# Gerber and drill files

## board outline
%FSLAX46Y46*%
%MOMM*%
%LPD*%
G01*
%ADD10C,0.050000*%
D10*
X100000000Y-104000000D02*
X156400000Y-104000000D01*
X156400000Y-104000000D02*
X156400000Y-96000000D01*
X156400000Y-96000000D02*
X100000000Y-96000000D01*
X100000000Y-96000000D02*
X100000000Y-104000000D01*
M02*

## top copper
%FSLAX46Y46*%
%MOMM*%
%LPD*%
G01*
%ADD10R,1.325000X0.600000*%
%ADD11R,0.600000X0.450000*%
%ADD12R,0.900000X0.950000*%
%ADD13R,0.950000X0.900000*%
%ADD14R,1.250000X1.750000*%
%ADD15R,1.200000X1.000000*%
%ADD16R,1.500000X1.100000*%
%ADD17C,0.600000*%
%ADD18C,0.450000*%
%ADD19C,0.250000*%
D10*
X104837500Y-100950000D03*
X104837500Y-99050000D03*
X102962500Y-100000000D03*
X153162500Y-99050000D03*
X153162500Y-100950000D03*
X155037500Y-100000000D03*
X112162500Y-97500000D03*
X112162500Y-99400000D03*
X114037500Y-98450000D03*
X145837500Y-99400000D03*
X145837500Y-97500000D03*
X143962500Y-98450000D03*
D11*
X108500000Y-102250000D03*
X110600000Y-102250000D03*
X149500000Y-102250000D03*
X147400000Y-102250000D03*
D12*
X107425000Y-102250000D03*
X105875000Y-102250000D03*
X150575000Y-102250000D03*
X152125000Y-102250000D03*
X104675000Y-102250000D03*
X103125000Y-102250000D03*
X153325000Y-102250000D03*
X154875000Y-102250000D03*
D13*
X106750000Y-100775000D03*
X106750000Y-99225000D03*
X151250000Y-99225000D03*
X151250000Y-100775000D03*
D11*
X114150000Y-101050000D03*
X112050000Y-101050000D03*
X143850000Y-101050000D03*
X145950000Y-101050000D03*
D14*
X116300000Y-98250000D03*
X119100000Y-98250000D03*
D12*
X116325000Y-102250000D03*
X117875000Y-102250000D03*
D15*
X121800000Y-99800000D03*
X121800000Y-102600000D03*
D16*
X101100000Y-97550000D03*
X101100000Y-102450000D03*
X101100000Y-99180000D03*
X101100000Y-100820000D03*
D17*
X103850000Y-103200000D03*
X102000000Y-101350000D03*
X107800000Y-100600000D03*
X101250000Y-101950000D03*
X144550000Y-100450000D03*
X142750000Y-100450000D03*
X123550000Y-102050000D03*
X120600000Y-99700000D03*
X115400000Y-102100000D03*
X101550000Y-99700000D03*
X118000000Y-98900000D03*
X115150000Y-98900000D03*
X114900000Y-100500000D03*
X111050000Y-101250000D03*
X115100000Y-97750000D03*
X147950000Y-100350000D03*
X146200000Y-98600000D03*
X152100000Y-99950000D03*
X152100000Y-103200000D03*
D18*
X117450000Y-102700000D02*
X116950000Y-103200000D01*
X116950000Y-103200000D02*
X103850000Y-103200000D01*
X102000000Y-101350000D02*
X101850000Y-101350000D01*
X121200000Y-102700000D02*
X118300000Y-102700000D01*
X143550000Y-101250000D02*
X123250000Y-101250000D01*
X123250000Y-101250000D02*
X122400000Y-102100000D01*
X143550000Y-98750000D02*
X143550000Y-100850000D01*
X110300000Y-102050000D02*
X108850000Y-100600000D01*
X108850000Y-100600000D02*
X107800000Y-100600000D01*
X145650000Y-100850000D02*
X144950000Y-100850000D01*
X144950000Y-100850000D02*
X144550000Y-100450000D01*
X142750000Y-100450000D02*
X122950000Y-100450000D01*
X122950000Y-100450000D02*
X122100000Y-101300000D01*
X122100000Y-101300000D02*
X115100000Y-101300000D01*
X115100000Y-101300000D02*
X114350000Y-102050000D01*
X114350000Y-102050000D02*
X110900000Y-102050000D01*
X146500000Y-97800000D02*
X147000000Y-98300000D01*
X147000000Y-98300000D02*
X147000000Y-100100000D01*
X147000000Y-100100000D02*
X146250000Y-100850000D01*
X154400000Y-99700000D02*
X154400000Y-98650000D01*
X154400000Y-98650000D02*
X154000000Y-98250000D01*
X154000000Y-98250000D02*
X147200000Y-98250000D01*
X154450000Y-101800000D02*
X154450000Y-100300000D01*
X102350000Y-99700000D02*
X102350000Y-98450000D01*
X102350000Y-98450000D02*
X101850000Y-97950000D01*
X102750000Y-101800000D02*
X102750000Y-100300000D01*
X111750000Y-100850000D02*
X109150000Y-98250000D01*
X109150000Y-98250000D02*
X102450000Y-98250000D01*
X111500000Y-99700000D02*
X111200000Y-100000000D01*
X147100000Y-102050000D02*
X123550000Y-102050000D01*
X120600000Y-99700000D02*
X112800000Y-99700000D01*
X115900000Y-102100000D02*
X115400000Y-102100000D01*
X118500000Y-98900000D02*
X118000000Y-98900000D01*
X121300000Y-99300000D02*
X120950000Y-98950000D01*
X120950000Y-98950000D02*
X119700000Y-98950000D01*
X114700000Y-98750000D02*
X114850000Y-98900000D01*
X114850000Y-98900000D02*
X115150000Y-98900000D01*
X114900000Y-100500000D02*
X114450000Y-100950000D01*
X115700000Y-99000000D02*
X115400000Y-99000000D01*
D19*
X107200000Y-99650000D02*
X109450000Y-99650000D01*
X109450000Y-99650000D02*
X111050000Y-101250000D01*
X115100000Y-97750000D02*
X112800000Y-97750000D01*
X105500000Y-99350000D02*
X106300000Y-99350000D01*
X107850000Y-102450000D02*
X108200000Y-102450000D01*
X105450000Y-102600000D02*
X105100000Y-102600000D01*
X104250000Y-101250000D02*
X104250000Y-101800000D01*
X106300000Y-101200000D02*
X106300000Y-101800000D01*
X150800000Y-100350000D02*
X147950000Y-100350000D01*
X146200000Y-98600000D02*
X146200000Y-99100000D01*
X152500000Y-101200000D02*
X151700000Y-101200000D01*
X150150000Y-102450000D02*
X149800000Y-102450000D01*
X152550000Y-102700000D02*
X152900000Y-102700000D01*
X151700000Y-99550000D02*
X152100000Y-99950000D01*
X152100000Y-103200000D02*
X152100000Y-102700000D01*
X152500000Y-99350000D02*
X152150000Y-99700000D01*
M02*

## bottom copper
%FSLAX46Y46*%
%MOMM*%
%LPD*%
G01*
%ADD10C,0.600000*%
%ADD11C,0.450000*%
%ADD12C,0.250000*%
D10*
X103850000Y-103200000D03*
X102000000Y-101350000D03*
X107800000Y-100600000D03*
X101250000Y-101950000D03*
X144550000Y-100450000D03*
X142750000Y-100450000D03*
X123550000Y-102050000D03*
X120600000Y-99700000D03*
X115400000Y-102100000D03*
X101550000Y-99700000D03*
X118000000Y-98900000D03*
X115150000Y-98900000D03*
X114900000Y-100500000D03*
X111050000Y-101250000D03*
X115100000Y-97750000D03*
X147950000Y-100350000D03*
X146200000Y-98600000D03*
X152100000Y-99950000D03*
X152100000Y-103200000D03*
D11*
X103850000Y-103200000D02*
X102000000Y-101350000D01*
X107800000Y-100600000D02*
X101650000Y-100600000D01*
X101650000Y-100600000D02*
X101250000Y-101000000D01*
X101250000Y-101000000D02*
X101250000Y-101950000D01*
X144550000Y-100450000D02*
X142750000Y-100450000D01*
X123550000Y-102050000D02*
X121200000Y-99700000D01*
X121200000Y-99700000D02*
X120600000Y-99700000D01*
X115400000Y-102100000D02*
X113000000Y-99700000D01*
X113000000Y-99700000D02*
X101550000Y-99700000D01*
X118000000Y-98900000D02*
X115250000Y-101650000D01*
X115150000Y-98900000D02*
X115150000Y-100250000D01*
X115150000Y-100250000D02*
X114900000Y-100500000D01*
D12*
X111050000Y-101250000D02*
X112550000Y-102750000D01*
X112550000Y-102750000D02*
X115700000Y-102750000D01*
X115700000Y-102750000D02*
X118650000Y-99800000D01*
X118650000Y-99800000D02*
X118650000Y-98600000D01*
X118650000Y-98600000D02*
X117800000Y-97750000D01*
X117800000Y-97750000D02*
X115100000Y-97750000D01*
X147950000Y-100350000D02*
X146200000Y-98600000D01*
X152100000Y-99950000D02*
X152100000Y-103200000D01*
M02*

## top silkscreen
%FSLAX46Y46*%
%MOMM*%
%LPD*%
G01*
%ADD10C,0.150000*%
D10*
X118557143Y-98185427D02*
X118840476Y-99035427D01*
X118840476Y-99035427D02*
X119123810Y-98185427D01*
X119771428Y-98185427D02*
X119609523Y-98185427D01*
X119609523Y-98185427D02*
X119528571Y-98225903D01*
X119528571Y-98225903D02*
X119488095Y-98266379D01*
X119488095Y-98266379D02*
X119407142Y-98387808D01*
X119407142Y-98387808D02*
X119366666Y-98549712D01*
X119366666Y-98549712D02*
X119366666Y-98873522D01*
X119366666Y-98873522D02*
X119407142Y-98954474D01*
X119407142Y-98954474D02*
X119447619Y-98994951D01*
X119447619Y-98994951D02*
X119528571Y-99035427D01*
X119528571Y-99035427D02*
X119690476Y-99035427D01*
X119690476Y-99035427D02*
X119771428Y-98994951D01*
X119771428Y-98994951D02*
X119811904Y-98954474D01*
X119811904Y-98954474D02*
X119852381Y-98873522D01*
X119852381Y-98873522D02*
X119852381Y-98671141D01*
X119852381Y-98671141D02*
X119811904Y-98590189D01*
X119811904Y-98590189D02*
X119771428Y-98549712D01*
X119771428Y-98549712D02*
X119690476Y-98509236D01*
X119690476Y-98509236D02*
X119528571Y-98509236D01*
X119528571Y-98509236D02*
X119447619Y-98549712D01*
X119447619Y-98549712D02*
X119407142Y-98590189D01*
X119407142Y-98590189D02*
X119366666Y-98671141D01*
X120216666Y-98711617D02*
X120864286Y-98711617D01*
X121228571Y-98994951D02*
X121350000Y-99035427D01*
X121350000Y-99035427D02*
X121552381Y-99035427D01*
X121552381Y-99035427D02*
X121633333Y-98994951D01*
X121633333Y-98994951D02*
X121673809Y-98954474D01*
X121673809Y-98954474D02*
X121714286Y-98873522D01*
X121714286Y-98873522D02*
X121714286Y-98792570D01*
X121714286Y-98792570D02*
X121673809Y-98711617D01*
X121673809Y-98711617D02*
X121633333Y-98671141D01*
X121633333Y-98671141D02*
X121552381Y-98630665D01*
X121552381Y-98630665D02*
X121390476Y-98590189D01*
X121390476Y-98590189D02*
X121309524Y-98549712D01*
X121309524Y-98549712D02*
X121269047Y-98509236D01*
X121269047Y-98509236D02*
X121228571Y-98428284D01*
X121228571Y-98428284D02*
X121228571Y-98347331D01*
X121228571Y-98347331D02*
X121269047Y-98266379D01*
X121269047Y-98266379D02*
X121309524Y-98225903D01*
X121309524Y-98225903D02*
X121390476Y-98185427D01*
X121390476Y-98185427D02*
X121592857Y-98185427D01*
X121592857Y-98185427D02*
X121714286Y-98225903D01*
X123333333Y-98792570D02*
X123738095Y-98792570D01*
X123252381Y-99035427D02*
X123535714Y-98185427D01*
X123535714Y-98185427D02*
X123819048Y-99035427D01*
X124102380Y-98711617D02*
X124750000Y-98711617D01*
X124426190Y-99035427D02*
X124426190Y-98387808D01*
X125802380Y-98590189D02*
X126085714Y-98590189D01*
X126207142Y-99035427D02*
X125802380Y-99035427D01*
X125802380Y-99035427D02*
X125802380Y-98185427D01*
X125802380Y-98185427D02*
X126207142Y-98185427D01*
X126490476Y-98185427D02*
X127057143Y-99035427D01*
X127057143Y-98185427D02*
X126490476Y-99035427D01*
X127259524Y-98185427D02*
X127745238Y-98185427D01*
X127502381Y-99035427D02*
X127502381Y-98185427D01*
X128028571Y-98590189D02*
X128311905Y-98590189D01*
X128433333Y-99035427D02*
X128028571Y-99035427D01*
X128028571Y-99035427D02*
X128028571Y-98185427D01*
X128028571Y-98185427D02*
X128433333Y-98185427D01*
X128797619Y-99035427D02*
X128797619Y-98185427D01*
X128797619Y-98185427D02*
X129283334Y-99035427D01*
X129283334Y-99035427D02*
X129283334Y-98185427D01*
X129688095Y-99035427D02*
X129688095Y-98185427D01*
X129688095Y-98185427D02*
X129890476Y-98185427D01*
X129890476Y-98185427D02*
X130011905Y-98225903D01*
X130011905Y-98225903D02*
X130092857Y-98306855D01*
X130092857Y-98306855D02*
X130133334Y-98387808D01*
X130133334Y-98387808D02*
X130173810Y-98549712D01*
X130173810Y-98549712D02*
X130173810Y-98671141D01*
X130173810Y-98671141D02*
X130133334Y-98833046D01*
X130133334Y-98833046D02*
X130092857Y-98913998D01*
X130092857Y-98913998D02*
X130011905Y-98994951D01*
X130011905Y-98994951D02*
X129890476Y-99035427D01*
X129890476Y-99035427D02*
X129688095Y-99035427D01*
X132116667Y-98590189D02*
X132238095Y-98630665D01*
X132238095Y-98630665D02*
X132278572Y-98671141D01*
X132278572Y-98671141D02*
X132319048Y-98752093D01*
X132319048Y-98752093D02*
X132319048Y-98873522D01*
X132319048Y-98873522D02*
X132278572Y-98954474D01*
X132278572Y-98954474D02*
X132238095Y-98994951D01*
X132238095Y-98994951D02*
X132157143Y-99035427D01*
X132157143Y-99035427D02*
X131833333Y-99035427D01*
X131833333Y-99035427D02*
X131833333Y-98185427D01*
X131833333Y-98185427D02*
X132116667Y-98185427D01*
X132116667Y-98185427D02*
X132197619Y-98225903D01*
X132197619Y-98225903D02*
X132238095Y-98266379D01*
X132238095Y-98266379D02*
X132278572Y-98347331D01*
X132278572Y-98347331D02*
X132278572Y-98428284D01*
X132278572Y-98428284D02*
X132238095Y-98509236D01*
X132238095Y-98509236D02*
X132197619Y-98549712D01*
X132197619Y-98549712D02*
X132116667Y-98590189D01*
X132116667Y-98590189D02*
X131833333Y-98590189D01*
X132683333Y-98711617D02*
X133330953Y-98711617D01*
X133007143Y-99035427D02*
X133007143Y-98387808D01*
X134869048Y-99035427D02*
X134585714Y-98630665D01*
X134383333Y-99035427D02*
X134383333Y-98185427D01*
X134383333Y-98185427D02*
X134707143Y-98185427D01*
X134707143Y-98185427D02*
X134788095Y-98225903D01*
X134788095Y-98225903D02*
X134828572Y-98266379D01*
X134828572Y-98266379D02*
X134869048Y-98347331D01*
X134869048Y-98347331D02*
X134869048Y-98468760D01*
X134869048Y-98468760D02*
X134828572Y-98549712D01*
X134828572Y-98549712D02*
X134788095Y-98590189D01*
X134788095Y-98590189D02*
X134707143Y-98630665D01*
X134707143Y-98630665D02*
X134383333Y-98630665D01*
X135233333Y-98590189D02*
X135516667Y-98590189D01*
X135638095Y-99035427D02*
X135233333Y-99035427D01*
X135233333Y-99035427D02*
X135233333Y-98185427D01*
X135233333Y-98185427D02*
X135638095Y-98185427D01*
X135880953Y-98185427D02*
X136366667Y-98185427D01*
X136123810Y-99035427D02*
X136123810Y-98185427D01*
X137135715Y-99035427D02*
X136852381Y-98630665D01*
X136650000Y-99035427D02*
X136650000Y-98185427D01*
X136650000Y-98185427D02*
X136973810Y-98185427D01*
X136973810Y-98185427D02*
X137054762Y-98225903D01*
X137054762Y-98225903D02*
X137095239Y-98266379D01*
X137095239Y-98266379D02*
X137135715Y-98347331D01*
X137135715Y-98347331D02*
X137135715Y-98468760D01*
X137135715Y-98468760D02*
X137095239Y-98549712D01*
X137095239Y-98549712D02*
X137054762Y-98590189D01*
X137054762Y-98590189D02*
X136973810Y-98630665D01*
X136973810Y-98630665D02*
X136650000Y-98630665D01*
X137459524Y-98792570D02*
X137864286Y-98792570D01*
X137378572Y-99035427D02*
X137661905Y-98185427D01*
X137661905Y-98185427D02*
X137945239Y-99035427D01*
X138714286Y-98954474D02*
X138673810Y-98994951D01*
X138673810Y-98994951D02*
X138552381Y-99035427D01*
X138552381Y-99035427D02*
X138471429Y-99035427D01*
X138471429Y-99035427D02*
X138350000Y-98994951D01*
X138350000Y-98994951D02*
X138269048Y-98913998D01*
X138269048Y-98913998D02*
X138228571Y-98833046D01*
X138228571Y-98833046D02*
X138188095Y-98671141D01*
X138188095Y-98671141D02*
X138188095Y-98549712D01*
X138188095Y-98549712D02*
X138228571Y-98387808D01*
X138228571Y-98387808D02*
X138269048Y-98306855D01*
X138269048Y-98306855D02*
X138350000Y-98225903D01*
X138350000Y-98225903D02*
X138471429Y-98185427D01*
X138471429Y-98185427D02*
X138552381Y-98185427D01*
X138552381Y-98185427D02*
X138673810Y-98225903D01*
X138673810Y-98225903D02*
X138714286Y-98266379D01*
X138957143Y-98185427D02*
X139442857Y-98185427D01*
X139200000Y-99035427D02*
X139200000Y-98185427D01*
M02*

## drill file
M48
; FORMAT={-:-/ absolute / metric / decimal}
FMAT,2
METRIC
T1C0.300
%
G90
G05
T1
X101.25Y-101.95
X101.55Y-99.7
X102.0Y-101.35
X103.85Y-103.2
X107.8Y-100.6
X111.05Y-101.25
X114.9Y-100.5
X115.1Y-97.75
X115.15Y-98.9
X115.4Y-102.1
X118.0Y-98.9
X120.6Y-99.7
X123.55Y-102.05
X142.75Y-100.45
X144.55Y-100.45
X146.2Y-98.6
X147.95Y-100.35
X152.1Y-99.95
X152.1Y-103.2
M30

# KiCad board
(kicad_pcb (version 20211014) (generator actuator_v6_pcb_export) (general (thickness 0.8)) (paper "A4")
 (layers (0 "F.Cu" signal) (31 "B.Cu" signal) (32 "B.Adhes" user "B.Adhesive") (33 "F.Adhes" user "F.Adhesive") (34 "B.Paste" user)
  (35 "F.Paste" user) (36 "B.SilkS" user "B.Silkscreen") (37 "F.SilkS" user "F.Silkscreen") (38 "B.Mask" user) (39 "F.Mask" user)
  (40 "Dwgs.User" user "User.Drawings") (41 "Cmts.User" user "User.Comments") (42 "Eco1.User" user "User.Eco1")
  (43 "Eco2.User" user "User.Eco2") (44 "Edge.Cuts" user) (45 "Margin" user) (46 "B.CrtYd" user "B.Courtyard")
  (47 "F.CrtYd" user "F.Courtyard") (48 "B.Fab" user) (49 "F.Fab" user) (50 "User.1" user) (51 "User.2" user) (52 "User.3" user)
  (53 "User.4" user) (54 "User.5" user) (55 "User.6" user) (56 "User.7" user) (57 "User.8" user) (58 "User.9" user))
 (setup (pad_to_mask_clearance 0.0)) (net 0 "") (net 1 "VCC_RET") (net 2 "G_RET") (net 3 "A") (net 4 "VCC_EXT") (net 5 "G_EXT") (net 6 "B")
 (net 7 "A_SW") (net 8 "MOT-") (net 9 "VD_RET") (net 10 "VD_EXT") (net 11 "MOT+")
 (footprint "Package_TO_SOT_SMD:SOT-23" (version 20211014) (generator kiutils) (layer "F.Cu") (at 103.9 100.0 180)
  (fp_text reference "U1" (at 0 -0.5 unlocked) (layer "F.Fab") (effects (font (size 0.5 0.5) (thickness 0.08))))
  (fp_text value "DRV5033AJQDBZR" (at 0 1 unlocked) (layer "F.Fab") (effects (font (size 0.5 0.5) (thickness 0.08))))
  (pad "1" smd rect (at -0.9375 -0.95 180) (size 1.325 0.6) (layers "F.Cu" "F.Mask" "F.Paste") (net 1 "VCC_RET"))
  (pad "2" smd rect (at -0.9375 0.95 180) (size 1.325 0.6) (layers "F.Cu" "F.Mask" "F.Paste") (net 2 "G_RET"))
  (pad "3" smd rect (at 0.9375 0.0 180) (size 1.325 0.6) (layers "F.Cu" "F.Mask" "F.Paste") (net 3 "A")))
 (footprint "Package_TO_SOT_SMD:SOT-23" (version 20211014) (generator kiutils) (layer "F.Cu") (at 154.1 100.0)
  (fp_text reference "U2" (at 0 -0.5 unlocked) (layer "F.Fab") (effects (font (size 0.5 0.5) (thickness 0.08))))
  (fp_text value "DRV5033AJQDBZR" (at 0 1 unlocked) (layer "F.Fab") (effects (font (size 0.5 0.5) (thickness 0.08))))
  (pad "1" smd rect (at -0.9375 -0.95) (size 1.325 0.6) (layers "F.Cu" "F.Mask" "F.Paste") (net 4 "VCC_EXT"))
  (pad "2" smd rect (at -0.9375 0.95) (size 1.325 0.6) (layers "F.Cu" "F.Mask" "F.Paste") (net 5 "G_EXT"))
  (pad "3" smd rect (at 0.9375 0.0) (size 1.325 0.6) (layers "F.Cu" "F.Mask" "F.Paste") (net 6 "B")))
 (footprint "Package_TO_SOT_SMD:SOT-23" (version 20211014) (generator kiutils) (layer "F.Cu") (at 113.1 98.45)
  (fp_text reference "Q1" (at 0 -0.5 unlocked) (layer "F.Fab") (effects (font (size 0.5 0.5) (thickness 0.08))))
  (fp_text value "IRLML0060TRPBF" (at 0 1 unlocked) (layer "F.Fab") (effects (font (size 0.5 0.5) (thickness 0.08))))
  (pad "1" smd rect (at -0.9375 -0.95) (size 1.325 0.6) (layers "F.Cu" "F.Mask" "F.Paste") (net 2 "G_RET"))
  (pad "2" smd rect (at -0.9375 0.95) (size 1.325 0.6) (layers "F.Cu" "F.Mask" "F.Paste") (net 3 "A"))
  (pad "3" smd rect (at 0.9375 0.0) (size 1.325 0.6) (layers "F.Cu" "F.Mask" "F.Paste") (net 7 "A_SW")))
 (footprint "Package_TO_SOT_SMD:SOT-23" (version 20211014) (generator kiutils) (layer "F.Cu") (at 144.9 98.45 180)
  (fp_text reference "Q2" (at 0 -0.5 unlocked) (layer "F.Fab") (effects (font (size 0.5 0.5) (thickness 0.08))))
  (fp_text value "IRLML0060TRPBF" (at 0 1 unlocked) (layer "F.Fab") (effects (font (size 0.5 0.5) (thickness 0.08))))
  (pad "1" smd rect (at -0.9375 -0.95 180) (size 1.325 0.6) (layers "F.Cu" "F.Mask" "F.Paste") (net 5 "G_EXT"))
  (pad "2" smd rect (at -0.9375 0.95 180) (size 1.325 0.6) (layers "F.Cu" "F.Mask" "F.Paste") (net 6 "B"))
  (pad "3" smd rect (at 0.9375 0.0 180) (size 1.325 0.6) (layers "F.Cu" "F.Mask" "F.Paste") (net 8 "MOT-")))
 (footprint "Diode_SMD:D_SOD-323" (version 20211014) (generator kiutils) (layer "F.Cu") (at 109.55 102.25)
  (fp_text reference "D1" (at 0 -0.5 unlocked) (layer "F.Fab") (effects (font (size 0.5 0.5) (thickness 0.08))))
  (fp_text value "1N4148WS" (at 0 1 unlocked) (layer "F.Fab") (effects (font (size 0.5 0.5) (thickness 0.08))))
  (pad "1" smd rect (at -1.05 0.0) (size 0.6 0.45) (layers "F.Cu" "F.Mask" "F.Paste") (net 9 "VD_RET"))
  (pad "2" smd rect (at 1.05 0.0) (size 0.6 0.45) (layers "F.Cu" "F.Mask" "F.Paste") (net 6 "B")))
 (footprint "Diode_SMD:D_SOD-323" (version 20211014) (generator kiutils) (layer "F.Cu") (at 148.45 102.25 180)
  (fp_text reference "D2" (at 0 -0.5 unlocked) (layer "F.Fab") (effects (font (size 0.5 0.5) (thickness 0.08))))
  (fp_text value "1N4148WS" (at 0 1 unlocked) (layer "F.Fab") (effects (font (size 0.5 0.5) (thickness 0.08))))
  (pad "1" smd rect (at -1.05 0.0 180) (size 0.6 0.45) (layers "F.Cu" "F.Mask" "F.Paste") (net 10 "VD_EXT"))
  (pad "2" smd rect (at 1.05 0.0 180) (size 0.6 0.45) (layers "F.Cu" "F.Mask" "F.Paste") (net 3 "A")))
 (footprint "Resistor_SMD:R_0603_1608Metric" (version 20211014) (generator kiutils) (layer "F.Cu") (at 106.65 102.25 180)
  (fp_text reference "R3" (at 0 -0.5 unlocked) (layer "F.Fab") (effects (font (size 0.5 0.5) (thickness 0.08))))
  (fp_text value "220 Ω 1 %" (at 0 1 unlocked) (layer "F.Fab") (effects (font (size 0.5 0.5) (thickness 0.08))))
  (pad "1" smd rect (at -0.775 0.0 180) (size 0.9 0.95) (layers "F.Cu" "F.Mask" "F.Paste") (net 9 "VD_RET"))
  (pad "2" smd rect (at 0.775 0.0 180) (size 0.9 0.95) (layers "F.Cu" "F.Mask" "F.Paste") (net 1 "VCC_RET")))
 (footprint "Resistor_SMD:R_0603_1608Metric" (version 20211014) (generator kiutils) (layer "F.Cu") (at 151.35 102.25)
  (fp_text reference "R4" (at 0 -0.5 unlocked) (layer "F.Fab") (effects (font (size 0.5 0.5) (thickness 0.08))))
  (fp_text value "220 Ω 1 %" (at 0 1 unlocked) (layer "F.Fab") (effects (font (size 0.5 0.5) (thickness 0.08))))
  (pad "1" smd rect (at -0.775 0.0) (size 0.9 0.95) (layers "F.Cu" "F.Mask" "F.Paste") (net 10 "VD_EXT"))
  (pad "2" smd rect (at 0.775 0.0) (size 0.9 0.95) (layers "F.Cu" "F.Mask" "F.Paste") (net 4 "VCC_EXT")))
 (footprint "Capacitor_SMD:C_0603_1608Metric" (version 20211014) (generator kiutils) (layer "F.Cu") (at 103.9 102.25 180)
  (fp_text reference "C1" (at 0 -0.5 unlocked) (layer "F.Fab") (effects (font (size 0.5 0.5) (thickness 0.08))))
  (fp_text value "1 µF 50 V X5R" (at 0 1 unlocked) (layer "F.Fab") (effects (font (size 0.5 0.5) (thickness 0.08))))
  (pad "1" smd rect (at -0.775 0.0 180) (size 0.9 0.95) (layers "F.Cu" "F.Mask" "F.Paste") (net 1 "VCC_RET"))
  (pad "2" smd rect (at 0.775 0.0 180) (size 0.9 0.95) (layers "F.Cu" "F.Mask" "F.Paste") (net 3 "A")))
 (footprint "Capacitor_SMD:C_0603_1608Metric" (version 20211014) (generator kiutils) (layer "F.Cu") (at 154.1 102.25)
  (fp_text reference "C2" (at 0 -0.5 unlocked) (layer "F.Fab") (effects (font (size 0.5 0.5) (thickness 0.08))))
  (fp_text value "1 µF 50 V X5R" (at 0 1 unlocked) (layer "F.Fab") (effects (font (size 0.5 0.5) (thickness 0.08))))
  (pad "1" smd rect (at -0.775 0.0) (size 0.9 0.95) (layers "F.Cu" "F.Mask" "F.Paste") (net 4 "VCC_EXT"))
  (pad "2" smd rect (at 0.775 0.0) (size 0.9 0.95) (layers "F.Cu" "F.Mask" "F.Paste") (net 6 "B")))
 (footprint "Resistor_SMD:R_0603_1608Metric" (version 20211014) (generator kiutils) (layer "F.Cu") (at 106.75 100.0 90)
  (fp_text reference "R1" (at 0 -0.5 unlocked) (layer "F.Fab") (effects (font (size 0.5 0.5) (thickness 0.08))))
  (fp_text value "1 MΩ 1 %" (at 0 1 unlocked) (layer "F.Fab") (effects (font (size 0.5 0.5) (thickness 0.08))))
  (pad "1" smd rect (at -0.775 0.0 90) (size 0.9 0.95) (layers "F.Cu" "F.Mask" "F.Paste") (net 1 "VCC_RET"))
  (pad "2" smd rect (at 0.775 0.0 90) (size 0.9 0.95) (layers "F.Cu" "F.Mask" "F.Paste") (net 2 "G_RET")))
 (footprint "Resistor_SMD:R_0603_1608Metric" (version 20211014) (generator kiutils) (layer "F.Cu") (at 151.25 100.0 270)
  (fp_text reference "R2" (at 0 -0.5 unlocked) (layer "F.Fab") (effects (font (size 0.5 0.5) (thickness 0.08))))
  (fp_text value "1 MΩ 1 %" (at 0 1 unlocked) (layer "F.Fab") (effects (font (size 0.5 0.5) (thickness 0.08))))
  (pad "1" smd rect (at -0.775 0.0 270) (size 0.9 0.95) (layers "F.Cu" "F.Mask" "F.Paste") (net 4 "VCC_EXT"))
  (pad "2" smd rect (at 0.775 0.0 270) (size 0.9 0.95) (layers "F.Cu" "F.Mask" "F.Paste") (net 5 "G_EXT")))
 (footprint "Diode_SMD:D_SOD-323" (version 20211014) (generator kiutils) (layer "F.Cu") (at 113.1 101.05 180)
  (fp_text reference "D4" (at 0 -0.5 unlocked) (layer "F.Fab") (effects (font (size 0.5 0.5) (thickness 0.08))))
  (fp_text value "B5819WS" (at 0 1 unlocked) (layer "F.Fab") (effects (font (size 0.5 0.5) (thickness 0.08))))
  (pad "1" smd rect (at -1.05 0.0 180) (size 0.6 0.45) (layers "F.Cu" "F.Mask" "F.Paste") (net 7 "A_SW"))
  (pad "2" smd rect (at 1.05 0.0 180) (size 0.6 0.45) (layers "F.Cu" "F.Mask" "F.Paste") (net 3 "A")))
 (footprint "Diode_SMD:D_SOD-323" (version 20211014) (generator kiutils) (layer "F.Cu") (at 144.9 101.05)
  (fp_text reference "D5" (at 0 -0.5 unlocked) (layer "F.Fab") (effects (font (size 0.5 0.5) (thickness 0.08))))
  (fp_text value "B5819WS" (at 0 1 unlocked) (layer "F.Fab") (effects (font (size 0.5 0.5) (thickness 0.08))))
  (pad "1" smd rect (at -1.05 0.0) (size 0.6 0.45) (layers "F.Cu" "F.Mask" "F.Paste") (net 8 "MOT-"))
  (pad "2" smd rect (at 1.05 0.0) (size 0.6 0.45) (layers "F.Cu" "F.Mask" "F.Paste") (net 6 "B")))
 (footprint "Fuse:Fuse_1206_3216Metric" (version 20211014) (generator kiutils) (layer "F.Cu") (at 117.7 98.25)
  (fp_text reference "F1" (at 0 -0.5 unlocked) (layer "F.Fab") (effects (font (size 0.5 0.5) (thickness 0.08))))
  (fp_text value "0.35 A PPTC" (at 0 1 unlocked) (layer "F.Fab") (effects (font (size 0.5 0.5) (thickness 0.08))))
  (pad "1" smd rect (at -1.4 0.0) (size 1.25 1.75) (layers "F.Cu" "F.Mask" "F.Paste") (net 7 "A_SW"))
  (pad "2" smd rect (at 1.4 0.0) (size 1.25 1.75) (layers "F.Cu" "F.Mask" "F.Paste") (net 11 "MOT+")))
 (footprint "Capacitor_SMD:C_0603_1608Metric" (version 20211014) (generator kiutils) (layer "F.Cu") (at 117.1 102.25)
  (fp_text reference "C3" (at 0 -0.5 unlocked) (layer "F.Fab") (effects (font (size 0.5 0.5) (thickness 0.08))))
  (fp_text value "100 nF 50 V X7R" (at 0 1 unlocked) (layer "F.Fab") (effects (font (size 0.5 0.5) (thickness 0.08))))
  (pad "1" smd rect (at -0.775 0.0) (size 0.9 0.95) (layers "F.Cu" "F.Mask" "F.Paste") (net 11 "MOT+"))
  (pad "2" smd rect (at 0.775 0.0) (size 0.9 0.95) (layers "F.Cu" "F.Mask" "F.Paste") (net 8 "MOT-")))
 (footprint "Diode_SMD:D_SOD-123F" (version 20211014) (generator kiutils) (layer "F.Cu") (at 121.8 101.2 270)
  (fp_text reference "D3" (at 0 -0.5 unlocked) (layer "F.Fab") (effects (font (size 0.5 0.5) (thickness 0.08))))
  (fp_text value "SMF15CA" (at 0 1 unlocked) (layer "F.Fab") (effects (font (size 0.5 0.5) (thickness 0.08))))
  (pad "1" smd rect (at -1.4 0.0 270) (size 1.0 1.2) (layers "F.Cu" "F.Mask" "F.Paste") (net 11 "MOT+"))
  (pad "2" smd rect (at 1.4 0.0 270) (size 1.0 1.2) (layers "F.Cu" "F.Mask" "F.Paste") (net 8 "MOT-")))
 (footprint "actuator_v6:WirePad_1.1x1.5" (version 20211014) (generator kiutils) (layer "F.Cu") (at 101.1 97.55)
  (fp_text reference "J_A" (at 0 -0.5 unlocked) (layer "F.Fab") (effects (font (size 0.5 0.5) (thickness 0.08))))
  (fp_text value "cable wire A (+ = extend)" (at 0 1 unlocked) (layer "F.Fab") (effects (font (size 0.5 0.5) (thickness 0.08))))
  (pad "1" smd rect (at 0.0 0.0) (size 1.5 1.1) (layers "F.Cu" "F.Mask") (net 3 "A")))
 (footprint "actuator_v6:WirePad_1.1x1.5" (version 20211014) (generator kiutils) (layer "F.Cu") (at 101.1 102.45)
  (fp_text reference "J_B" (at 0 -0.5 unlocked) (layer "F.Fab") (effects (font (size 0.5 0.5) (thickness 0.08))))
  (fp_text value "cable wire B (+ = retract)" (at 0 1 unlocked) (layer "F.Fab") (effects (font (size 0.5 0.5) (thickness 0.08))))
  (pad "1" smd rect (at 0.0 0.0) (size 1.5 1.1) (layers "F.Cu" "F.Mask") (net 6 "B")))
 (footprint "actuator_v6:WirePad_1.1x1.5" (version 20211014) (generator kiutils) (layer "F.Cu") (at 101.1 99.18)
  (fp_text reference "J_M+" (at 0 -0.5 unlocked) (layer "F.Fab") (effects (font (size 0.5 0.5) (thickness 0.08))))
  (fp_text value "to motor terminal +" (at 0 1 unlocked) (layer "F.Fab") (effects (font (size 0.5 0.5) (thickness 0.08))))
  (pad "1" smd rect (at 0.0 0.0) (size 1.5 1.1) (layers "F.Cu" "F.Mask") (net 11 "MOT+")))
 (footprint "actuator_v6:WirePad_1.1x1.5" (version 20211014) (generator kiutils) (layer "F.Cu") (at 101.1 100.82)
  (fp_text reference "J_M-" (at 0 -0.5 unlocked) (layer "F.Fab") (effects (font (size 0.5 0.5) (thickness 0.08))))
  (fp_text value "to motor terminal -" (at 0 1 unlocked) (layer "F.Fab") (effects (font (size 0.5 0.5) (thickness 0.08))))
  (pad "1" smd rect (at 0.0 0.0) (size 1.5 1.1) (layers "F.Cu" "F.Mask") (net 8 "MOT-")))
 (gr_line (start 100.0 104.0) (end 156.4 104.0) (layer "Edge.Cuts") (width 0.05))
 (gr_line (start 156.4 104.0) (end 156.4 96.0) (layer "Edge.Cuts") (width 0.05))
 (gr_line (start 156.4 96.0) (end 100.0 96.0) (layer "Edge.Cuts") (width 0.05))
 (gr_line (start 100.0 96.0) (end 100.0 104.0) (layer "Edge.Cuts") (width 0.05))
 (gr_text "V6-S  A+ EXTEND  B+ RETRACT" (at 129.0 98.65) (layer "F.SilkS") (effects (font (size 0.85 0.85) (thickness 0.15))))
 (segment (start 117.45 102.7) (end 116.95 103.2) (width 0.45) (layer "F.Cu") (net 8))
 (segment (start 116.95 103.2) (end 103.85 103.2) (width 0.45) (layer "F.Cu") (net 8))
 (segment (start 103.85 103.2) (end 102.0 101.35) (width 0.45) (layer "B.Cu") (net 8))
 (segment (start 102.0 101.35) (end 101.85 101.35) (width 0.45) (layer "F.Cu") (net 8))
 (segment (start 121.2 102.7) (end 118.3 102.7) (width 0.45) (layer "F.Cu") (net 8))
 (segment (start 143.55 101.25) (end 123.25 101.25) (width 0.45) (layer "F.Cu") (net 8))
 (segment (start 123.25 101.25) (end 122.4 102.1) (width 0.45) (layer "F.Cu") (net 8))
 (segment (start 143.55 98.75) (end 143.55 100.85) (width 0.45) (layer "F.Cu") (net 8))
 (segment (start 110.3 102.05) (end 108.85 100.6) (width 0.45) (layer "F.Cu") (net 6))
 (segment (start 108.85 100.6) (end 107.8 100.6) (width 0.45) (layer "F.Cu") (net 6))
 (segment (start 107.8 100.6) (end 101.65 100.6) (width 0.45) (layer "B.Cu") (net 6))
 (segment (start 101.65 100.6) (end 101.25 101.0) (width 0.45) (layer "B.Cu") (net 6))
 (segment (start 101.25 101.0) (end 101.25 101.95) (width 0.45) (layer "B.Cu") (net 6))
 (segment (start 145.65 100.85) (end 144.95 100.85) (width 0.45) (layer "F.Cu") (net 6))
 (segment (start 144.95 100.85) (end 144.55 100.45) (width 0.45) (layer "F.Cu") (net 6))
 (segment (start 144.55 100.45) (end 142.75 100.45) (width 0.45) (layer "B.Cu") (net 6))
 (segment (start 142.75 100.45) (end 122.95 100.45) (width 0.45) (layer "F.Cu") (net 6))
 (segment (start 122.95 100.45) (end 122.1 101.3) (width 0.45) (layer "F.Cu") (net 6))
 (segment (start 122.1 101.3) (end 115.1 101.3) (width 0.45) (layer "F.Cu") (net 6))
 (segment (start 115.1 101.3) (end 114.35 102.05) (width 0.45) (layer "F.Cu") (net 6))
 (segment (start 114.35 102.05) (end 110.9 102.05) (width 0.45) (layer "F.Cu") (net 6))
 (segment (start 146.5 97.8) (end 147.0 98.3) (width 0.45) (layer "F.Cu") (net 6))
 (segment (start 147.0 98.3) (end 147.0 100.1) (width 0.45) (layer "F.Cu") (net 6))
 (segment (start 147.0 100.1) (end 146.25 100.85) (width 0.45) (layer "F.Cu") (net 6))
 (segment (start 154.4 99.7) (end 154.4 98.65) (width 0.45) (layer "F.Cu") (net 6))
 (segment (start 154.4 98.65) (end 154.0 98.25) (width 0.45) (layer "F.Cu") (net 6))
 (segment (start 154.0 98.25) (end 147.2 98.25) (width 0.45) (layer "F.Cu") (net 6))
 (segment (start 154.45 101.8) (end 154.45 100.3) (width 0.45) (layer "F.Cu") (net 6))
 (segment (start 102.35 99.7) (end 102.35 98.45) (width 0.45) (layer "F.Cu") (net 3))
 (segment (start 102.35 98.45) (end 101.85 97.95) (width 0.45) (layer "F.Cu") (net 3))
 (segment (start 102.75 101.8) (end 102.75 100.3) (width 0.45) (layer "F.Cu") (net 3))
 (segment (start 111.75 100.85) (end 109.15 98.25) (width 0.45) (layer "F.Cu") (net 3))
 (segment (start 109.15 98.25) (end 102.45 98.25) (width 0.45) (layer "F.Cu") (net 3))
 (segment (start 111.5 99.7) (end 111.2 100.0) (width 0.45) (layer "F.Cu") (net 3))
 (segment (start 147.1 102.05) (end 123.55 102.05) (width 0.45) (layer "F.Cu") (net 3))
 (segment (start 123.55 102.05) (end 121.2 99.7) (width 0.45) (layer "B.Cu") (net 3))
 (segment (start 121.2 99.7) (end 120.6 99.7) (width 0.45) (layer "B.Cu") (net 3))
 (segment (start 120.6 99.7) (end 112.8 99.7) (width 0.45) (layer "F.Cu") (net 3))
 (segment (start 115.9 102.1) (end 115.4 102.1) (width 0.45) (layer "F.Cu") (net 11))
 (segment (start 115.4 102.1) (end 113.0 99.7) (width 0.45) (layer "B.Cu") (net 11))
 (segment (start 113.0 99.7) (end 101.55 99.7) (width 0.45) (layer "B.Cu") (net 11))
 (segment (start 118.5 98.9) (end 118.0 98.9) (width 0.45) (layer "F.Cu") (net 11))
 (segment (start 118.0 98.9) (end 115.25 101.65) (width 0.45) (layer "B.Cu") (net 11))
 (segment (start 121.3 99.3) (end 120.95 98.95) (width 0.45) (layer "F.Cu") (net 11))
 (segment (start 120.95 98.95) (end 119.7 98.95) (width 0.45) (layer "F.Cu") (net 11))
 (segment (start 114.7 98.75) (end 114.85 98.9) (width 0.45) (layer "F.Cu") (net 7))
 (segment (start 114.85 98.9) (end 115.15 98.9) (width 0.45) (layer "F.Cu") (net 7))
 (segment (start 115.15 98.9) (end 115.15 100.25) (width 0.45) (layer "B.Cu") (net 7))
 (segment (start 115.15 100.25) (end 114.9 100.5) (width 0.45) (layer "B.Cu") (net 7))
 (segment (start 114.9 100.5) (end 114.45 100.95) (width 0.45) (layer "F.Cu") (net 7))
 (segment (start 115.7 99.0) (end 115.4 99.0) (width 0.45) (layer "F.Cu") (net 7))
 (segment (start 107.2 99.65) (end 109.45 99.65) (width 0.25) (layer "F.Cu") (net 2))
 (segment (start 109.45 99.65) (end 111.05 101.25) (width 0.25) (layer "F.Cu") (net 2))
 (segment (start 111.05 101.25) (end 112.55 102.75) (width 0.25) (layer "B.Cu") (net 2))
 (segment (start 112.55 102.75) (end 115.7 102.75) (width 0.25) (layer "B.Cu") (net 2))
 (segment (start 115.7 102.75) (end 118.65 99.8) (width 0.25) (layer "B.Cu") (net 2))
 (segment (start 118.65 99.8) (end 118.65 98.6) (width 0.25) (layer "B.Cu") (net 2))
 (segment (start 118.65 98.6) (end 117.8 97.75) (width 0.25) (layer "B.Cu") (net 2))
 (segment (start 117.8 97.75) (end 115.1 97.75) (width 0.25) (layer "B.Cu") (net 2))
 (segment (start 115.1 97.75) (end 112.8 97.75) (width 0.25) (layer "F.Cu") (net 2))
 (segment (start 105.5 99.35) (end 106.3 99.35) (width 0.25) (layer "F.Cu") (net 2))
 (segment (start 107.85 102.45) (end 108.2 102.45) (width 0.25) (layer "F.Cu") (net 9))
 (segment (start 105.45 102.6) (end 105.1 102.6) (width 0.25) (layer "F.Cu") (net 1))
 (segment (start 104.25 101.25) (end 104.25 101.8) (width 0.25) (layer "F.Cu") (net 1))
 (segment (start 106.3 101.2) (end 106.3 101.8) (width 0.25) (layer "F.Cu") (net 1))
 (segment (start 150.8 100.35) (end 147.95 100.35) (width 0.25) (layer "F.Cu") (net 5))
 (segment (start 147.95 100.35) (end 146.2 98.6) (width 0.25) (layer "B.Cu") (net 5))
 (segment (start 146.2 98.6) (end 146.2 99.1) (width 0.25) (layer "F.Cu") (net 5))
 (segment (start 152.5 101.2) (end 151.7 101.2) (width 0.25) (layer "F.Cu") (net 5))
 (segment (start 150.15 102.45) (end 149.8 102.45) (width 0.25) (layer "F.Cu") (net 10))
 (segment (start 152.55 102.7) (end 152.9 102.7) (width 0.25) (layer "F.Cu") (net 4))
 (segment (start 151.7 99.55) (end 152.1 99.95) (width 0.25) (layer "F.Cu") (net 4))
 (segment (start 152.1 99.95) (end 152.1 103.2) (width 0.25) (layer "B.Cu") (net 4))
 (segment (start 152.1 103.2) (end 152.1 102.7) (width 0.25) (layer "F.Cu") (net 4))
 (segment (start 152.5 99.35) (end 152.15 99.7) (width 0.25) (layer "F.Cu") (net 4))
 (via (at 103.85 103.2) (size 0.6) (drill 0.3) (layers "F.Cu" "B.Cu") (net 8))
 (via (at 102.0 101.35) (size 0.6) (drill 0.3) (layers "F.Cu" "B.Cu") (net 8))
 (via (at 107.8 100.6) (size 0.6) (drill 0.3) (layers "F.Cu" "B.Cu") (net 6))
 (via (at 101.25 101.95) (size 0.6) (drill 0.3) (layers "F.Cu" "B.Cu") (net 6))
 (via (at 144.55 100.45) (size 0.6) (drill 0.3) (layers "F.Cu" "B.Cu") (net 6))
 (via (at 142.75 100.45) (size 0.6) (drill 0.3) (layers "F.Cu" "B.Cu") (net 6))
 (via (at 123.55 102.05) (size 0.6) (drill 0.3) (layers "F.Cu" "B.Cu") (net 3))
 (via (at 120.6 99.7) (size 0.6) (drill 0.3) (layers "F.Cu" "B.Cu") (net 3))
 (via (at 115.4 102.1) (size 0.6) (drill 0.3) (layers "F.Cu" "B.Cu") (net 11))
 (via (at 101.55 99.7) (size 0.6) (drill 0.3) (layers "F.Cu" "B.Cu") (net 11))
 (via (at 118.0 98.9) (size 0.6) (drill 0.3) (layers "F.Cu" "B.Cu") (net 11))
 (via (at 115.15 98.9) (size 0.6) (drill 0.3) (layers "F.Cu" "B.Cu") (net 7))
 (via (at 114.9 100.5) (size 0.6) (drill 0.3) (layers "F.Cu" "B.Cu") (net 7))
 (via (at 111.05 101.25) (size 0.6) (drill 0.3) (layers "F.Cu" "B.Cu") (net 2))
 (via (at 115.1 97.75) (size 0.6) (drill 0.3) (layers "F.Cu" "B.Cu") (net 2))
 (via (at 147.95 100.35) (size 0.6) (drill 0.3) (layers "F.Cu" "B.Cu") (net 5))
 (via (at 146.2 98.6) (size 0.6) (drill 0.3) (layers "F.Cu" "B.Cu") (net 5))
 (via (at 152.1 99.95) (size 0.6) (drill 0.3) (layers "F.Cu" "B.Cu") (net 4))
 (via (at 152.1 103.2) (size 0.6) (drill 0.3) (layers "F.Cu" "B.Cu") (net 4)))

